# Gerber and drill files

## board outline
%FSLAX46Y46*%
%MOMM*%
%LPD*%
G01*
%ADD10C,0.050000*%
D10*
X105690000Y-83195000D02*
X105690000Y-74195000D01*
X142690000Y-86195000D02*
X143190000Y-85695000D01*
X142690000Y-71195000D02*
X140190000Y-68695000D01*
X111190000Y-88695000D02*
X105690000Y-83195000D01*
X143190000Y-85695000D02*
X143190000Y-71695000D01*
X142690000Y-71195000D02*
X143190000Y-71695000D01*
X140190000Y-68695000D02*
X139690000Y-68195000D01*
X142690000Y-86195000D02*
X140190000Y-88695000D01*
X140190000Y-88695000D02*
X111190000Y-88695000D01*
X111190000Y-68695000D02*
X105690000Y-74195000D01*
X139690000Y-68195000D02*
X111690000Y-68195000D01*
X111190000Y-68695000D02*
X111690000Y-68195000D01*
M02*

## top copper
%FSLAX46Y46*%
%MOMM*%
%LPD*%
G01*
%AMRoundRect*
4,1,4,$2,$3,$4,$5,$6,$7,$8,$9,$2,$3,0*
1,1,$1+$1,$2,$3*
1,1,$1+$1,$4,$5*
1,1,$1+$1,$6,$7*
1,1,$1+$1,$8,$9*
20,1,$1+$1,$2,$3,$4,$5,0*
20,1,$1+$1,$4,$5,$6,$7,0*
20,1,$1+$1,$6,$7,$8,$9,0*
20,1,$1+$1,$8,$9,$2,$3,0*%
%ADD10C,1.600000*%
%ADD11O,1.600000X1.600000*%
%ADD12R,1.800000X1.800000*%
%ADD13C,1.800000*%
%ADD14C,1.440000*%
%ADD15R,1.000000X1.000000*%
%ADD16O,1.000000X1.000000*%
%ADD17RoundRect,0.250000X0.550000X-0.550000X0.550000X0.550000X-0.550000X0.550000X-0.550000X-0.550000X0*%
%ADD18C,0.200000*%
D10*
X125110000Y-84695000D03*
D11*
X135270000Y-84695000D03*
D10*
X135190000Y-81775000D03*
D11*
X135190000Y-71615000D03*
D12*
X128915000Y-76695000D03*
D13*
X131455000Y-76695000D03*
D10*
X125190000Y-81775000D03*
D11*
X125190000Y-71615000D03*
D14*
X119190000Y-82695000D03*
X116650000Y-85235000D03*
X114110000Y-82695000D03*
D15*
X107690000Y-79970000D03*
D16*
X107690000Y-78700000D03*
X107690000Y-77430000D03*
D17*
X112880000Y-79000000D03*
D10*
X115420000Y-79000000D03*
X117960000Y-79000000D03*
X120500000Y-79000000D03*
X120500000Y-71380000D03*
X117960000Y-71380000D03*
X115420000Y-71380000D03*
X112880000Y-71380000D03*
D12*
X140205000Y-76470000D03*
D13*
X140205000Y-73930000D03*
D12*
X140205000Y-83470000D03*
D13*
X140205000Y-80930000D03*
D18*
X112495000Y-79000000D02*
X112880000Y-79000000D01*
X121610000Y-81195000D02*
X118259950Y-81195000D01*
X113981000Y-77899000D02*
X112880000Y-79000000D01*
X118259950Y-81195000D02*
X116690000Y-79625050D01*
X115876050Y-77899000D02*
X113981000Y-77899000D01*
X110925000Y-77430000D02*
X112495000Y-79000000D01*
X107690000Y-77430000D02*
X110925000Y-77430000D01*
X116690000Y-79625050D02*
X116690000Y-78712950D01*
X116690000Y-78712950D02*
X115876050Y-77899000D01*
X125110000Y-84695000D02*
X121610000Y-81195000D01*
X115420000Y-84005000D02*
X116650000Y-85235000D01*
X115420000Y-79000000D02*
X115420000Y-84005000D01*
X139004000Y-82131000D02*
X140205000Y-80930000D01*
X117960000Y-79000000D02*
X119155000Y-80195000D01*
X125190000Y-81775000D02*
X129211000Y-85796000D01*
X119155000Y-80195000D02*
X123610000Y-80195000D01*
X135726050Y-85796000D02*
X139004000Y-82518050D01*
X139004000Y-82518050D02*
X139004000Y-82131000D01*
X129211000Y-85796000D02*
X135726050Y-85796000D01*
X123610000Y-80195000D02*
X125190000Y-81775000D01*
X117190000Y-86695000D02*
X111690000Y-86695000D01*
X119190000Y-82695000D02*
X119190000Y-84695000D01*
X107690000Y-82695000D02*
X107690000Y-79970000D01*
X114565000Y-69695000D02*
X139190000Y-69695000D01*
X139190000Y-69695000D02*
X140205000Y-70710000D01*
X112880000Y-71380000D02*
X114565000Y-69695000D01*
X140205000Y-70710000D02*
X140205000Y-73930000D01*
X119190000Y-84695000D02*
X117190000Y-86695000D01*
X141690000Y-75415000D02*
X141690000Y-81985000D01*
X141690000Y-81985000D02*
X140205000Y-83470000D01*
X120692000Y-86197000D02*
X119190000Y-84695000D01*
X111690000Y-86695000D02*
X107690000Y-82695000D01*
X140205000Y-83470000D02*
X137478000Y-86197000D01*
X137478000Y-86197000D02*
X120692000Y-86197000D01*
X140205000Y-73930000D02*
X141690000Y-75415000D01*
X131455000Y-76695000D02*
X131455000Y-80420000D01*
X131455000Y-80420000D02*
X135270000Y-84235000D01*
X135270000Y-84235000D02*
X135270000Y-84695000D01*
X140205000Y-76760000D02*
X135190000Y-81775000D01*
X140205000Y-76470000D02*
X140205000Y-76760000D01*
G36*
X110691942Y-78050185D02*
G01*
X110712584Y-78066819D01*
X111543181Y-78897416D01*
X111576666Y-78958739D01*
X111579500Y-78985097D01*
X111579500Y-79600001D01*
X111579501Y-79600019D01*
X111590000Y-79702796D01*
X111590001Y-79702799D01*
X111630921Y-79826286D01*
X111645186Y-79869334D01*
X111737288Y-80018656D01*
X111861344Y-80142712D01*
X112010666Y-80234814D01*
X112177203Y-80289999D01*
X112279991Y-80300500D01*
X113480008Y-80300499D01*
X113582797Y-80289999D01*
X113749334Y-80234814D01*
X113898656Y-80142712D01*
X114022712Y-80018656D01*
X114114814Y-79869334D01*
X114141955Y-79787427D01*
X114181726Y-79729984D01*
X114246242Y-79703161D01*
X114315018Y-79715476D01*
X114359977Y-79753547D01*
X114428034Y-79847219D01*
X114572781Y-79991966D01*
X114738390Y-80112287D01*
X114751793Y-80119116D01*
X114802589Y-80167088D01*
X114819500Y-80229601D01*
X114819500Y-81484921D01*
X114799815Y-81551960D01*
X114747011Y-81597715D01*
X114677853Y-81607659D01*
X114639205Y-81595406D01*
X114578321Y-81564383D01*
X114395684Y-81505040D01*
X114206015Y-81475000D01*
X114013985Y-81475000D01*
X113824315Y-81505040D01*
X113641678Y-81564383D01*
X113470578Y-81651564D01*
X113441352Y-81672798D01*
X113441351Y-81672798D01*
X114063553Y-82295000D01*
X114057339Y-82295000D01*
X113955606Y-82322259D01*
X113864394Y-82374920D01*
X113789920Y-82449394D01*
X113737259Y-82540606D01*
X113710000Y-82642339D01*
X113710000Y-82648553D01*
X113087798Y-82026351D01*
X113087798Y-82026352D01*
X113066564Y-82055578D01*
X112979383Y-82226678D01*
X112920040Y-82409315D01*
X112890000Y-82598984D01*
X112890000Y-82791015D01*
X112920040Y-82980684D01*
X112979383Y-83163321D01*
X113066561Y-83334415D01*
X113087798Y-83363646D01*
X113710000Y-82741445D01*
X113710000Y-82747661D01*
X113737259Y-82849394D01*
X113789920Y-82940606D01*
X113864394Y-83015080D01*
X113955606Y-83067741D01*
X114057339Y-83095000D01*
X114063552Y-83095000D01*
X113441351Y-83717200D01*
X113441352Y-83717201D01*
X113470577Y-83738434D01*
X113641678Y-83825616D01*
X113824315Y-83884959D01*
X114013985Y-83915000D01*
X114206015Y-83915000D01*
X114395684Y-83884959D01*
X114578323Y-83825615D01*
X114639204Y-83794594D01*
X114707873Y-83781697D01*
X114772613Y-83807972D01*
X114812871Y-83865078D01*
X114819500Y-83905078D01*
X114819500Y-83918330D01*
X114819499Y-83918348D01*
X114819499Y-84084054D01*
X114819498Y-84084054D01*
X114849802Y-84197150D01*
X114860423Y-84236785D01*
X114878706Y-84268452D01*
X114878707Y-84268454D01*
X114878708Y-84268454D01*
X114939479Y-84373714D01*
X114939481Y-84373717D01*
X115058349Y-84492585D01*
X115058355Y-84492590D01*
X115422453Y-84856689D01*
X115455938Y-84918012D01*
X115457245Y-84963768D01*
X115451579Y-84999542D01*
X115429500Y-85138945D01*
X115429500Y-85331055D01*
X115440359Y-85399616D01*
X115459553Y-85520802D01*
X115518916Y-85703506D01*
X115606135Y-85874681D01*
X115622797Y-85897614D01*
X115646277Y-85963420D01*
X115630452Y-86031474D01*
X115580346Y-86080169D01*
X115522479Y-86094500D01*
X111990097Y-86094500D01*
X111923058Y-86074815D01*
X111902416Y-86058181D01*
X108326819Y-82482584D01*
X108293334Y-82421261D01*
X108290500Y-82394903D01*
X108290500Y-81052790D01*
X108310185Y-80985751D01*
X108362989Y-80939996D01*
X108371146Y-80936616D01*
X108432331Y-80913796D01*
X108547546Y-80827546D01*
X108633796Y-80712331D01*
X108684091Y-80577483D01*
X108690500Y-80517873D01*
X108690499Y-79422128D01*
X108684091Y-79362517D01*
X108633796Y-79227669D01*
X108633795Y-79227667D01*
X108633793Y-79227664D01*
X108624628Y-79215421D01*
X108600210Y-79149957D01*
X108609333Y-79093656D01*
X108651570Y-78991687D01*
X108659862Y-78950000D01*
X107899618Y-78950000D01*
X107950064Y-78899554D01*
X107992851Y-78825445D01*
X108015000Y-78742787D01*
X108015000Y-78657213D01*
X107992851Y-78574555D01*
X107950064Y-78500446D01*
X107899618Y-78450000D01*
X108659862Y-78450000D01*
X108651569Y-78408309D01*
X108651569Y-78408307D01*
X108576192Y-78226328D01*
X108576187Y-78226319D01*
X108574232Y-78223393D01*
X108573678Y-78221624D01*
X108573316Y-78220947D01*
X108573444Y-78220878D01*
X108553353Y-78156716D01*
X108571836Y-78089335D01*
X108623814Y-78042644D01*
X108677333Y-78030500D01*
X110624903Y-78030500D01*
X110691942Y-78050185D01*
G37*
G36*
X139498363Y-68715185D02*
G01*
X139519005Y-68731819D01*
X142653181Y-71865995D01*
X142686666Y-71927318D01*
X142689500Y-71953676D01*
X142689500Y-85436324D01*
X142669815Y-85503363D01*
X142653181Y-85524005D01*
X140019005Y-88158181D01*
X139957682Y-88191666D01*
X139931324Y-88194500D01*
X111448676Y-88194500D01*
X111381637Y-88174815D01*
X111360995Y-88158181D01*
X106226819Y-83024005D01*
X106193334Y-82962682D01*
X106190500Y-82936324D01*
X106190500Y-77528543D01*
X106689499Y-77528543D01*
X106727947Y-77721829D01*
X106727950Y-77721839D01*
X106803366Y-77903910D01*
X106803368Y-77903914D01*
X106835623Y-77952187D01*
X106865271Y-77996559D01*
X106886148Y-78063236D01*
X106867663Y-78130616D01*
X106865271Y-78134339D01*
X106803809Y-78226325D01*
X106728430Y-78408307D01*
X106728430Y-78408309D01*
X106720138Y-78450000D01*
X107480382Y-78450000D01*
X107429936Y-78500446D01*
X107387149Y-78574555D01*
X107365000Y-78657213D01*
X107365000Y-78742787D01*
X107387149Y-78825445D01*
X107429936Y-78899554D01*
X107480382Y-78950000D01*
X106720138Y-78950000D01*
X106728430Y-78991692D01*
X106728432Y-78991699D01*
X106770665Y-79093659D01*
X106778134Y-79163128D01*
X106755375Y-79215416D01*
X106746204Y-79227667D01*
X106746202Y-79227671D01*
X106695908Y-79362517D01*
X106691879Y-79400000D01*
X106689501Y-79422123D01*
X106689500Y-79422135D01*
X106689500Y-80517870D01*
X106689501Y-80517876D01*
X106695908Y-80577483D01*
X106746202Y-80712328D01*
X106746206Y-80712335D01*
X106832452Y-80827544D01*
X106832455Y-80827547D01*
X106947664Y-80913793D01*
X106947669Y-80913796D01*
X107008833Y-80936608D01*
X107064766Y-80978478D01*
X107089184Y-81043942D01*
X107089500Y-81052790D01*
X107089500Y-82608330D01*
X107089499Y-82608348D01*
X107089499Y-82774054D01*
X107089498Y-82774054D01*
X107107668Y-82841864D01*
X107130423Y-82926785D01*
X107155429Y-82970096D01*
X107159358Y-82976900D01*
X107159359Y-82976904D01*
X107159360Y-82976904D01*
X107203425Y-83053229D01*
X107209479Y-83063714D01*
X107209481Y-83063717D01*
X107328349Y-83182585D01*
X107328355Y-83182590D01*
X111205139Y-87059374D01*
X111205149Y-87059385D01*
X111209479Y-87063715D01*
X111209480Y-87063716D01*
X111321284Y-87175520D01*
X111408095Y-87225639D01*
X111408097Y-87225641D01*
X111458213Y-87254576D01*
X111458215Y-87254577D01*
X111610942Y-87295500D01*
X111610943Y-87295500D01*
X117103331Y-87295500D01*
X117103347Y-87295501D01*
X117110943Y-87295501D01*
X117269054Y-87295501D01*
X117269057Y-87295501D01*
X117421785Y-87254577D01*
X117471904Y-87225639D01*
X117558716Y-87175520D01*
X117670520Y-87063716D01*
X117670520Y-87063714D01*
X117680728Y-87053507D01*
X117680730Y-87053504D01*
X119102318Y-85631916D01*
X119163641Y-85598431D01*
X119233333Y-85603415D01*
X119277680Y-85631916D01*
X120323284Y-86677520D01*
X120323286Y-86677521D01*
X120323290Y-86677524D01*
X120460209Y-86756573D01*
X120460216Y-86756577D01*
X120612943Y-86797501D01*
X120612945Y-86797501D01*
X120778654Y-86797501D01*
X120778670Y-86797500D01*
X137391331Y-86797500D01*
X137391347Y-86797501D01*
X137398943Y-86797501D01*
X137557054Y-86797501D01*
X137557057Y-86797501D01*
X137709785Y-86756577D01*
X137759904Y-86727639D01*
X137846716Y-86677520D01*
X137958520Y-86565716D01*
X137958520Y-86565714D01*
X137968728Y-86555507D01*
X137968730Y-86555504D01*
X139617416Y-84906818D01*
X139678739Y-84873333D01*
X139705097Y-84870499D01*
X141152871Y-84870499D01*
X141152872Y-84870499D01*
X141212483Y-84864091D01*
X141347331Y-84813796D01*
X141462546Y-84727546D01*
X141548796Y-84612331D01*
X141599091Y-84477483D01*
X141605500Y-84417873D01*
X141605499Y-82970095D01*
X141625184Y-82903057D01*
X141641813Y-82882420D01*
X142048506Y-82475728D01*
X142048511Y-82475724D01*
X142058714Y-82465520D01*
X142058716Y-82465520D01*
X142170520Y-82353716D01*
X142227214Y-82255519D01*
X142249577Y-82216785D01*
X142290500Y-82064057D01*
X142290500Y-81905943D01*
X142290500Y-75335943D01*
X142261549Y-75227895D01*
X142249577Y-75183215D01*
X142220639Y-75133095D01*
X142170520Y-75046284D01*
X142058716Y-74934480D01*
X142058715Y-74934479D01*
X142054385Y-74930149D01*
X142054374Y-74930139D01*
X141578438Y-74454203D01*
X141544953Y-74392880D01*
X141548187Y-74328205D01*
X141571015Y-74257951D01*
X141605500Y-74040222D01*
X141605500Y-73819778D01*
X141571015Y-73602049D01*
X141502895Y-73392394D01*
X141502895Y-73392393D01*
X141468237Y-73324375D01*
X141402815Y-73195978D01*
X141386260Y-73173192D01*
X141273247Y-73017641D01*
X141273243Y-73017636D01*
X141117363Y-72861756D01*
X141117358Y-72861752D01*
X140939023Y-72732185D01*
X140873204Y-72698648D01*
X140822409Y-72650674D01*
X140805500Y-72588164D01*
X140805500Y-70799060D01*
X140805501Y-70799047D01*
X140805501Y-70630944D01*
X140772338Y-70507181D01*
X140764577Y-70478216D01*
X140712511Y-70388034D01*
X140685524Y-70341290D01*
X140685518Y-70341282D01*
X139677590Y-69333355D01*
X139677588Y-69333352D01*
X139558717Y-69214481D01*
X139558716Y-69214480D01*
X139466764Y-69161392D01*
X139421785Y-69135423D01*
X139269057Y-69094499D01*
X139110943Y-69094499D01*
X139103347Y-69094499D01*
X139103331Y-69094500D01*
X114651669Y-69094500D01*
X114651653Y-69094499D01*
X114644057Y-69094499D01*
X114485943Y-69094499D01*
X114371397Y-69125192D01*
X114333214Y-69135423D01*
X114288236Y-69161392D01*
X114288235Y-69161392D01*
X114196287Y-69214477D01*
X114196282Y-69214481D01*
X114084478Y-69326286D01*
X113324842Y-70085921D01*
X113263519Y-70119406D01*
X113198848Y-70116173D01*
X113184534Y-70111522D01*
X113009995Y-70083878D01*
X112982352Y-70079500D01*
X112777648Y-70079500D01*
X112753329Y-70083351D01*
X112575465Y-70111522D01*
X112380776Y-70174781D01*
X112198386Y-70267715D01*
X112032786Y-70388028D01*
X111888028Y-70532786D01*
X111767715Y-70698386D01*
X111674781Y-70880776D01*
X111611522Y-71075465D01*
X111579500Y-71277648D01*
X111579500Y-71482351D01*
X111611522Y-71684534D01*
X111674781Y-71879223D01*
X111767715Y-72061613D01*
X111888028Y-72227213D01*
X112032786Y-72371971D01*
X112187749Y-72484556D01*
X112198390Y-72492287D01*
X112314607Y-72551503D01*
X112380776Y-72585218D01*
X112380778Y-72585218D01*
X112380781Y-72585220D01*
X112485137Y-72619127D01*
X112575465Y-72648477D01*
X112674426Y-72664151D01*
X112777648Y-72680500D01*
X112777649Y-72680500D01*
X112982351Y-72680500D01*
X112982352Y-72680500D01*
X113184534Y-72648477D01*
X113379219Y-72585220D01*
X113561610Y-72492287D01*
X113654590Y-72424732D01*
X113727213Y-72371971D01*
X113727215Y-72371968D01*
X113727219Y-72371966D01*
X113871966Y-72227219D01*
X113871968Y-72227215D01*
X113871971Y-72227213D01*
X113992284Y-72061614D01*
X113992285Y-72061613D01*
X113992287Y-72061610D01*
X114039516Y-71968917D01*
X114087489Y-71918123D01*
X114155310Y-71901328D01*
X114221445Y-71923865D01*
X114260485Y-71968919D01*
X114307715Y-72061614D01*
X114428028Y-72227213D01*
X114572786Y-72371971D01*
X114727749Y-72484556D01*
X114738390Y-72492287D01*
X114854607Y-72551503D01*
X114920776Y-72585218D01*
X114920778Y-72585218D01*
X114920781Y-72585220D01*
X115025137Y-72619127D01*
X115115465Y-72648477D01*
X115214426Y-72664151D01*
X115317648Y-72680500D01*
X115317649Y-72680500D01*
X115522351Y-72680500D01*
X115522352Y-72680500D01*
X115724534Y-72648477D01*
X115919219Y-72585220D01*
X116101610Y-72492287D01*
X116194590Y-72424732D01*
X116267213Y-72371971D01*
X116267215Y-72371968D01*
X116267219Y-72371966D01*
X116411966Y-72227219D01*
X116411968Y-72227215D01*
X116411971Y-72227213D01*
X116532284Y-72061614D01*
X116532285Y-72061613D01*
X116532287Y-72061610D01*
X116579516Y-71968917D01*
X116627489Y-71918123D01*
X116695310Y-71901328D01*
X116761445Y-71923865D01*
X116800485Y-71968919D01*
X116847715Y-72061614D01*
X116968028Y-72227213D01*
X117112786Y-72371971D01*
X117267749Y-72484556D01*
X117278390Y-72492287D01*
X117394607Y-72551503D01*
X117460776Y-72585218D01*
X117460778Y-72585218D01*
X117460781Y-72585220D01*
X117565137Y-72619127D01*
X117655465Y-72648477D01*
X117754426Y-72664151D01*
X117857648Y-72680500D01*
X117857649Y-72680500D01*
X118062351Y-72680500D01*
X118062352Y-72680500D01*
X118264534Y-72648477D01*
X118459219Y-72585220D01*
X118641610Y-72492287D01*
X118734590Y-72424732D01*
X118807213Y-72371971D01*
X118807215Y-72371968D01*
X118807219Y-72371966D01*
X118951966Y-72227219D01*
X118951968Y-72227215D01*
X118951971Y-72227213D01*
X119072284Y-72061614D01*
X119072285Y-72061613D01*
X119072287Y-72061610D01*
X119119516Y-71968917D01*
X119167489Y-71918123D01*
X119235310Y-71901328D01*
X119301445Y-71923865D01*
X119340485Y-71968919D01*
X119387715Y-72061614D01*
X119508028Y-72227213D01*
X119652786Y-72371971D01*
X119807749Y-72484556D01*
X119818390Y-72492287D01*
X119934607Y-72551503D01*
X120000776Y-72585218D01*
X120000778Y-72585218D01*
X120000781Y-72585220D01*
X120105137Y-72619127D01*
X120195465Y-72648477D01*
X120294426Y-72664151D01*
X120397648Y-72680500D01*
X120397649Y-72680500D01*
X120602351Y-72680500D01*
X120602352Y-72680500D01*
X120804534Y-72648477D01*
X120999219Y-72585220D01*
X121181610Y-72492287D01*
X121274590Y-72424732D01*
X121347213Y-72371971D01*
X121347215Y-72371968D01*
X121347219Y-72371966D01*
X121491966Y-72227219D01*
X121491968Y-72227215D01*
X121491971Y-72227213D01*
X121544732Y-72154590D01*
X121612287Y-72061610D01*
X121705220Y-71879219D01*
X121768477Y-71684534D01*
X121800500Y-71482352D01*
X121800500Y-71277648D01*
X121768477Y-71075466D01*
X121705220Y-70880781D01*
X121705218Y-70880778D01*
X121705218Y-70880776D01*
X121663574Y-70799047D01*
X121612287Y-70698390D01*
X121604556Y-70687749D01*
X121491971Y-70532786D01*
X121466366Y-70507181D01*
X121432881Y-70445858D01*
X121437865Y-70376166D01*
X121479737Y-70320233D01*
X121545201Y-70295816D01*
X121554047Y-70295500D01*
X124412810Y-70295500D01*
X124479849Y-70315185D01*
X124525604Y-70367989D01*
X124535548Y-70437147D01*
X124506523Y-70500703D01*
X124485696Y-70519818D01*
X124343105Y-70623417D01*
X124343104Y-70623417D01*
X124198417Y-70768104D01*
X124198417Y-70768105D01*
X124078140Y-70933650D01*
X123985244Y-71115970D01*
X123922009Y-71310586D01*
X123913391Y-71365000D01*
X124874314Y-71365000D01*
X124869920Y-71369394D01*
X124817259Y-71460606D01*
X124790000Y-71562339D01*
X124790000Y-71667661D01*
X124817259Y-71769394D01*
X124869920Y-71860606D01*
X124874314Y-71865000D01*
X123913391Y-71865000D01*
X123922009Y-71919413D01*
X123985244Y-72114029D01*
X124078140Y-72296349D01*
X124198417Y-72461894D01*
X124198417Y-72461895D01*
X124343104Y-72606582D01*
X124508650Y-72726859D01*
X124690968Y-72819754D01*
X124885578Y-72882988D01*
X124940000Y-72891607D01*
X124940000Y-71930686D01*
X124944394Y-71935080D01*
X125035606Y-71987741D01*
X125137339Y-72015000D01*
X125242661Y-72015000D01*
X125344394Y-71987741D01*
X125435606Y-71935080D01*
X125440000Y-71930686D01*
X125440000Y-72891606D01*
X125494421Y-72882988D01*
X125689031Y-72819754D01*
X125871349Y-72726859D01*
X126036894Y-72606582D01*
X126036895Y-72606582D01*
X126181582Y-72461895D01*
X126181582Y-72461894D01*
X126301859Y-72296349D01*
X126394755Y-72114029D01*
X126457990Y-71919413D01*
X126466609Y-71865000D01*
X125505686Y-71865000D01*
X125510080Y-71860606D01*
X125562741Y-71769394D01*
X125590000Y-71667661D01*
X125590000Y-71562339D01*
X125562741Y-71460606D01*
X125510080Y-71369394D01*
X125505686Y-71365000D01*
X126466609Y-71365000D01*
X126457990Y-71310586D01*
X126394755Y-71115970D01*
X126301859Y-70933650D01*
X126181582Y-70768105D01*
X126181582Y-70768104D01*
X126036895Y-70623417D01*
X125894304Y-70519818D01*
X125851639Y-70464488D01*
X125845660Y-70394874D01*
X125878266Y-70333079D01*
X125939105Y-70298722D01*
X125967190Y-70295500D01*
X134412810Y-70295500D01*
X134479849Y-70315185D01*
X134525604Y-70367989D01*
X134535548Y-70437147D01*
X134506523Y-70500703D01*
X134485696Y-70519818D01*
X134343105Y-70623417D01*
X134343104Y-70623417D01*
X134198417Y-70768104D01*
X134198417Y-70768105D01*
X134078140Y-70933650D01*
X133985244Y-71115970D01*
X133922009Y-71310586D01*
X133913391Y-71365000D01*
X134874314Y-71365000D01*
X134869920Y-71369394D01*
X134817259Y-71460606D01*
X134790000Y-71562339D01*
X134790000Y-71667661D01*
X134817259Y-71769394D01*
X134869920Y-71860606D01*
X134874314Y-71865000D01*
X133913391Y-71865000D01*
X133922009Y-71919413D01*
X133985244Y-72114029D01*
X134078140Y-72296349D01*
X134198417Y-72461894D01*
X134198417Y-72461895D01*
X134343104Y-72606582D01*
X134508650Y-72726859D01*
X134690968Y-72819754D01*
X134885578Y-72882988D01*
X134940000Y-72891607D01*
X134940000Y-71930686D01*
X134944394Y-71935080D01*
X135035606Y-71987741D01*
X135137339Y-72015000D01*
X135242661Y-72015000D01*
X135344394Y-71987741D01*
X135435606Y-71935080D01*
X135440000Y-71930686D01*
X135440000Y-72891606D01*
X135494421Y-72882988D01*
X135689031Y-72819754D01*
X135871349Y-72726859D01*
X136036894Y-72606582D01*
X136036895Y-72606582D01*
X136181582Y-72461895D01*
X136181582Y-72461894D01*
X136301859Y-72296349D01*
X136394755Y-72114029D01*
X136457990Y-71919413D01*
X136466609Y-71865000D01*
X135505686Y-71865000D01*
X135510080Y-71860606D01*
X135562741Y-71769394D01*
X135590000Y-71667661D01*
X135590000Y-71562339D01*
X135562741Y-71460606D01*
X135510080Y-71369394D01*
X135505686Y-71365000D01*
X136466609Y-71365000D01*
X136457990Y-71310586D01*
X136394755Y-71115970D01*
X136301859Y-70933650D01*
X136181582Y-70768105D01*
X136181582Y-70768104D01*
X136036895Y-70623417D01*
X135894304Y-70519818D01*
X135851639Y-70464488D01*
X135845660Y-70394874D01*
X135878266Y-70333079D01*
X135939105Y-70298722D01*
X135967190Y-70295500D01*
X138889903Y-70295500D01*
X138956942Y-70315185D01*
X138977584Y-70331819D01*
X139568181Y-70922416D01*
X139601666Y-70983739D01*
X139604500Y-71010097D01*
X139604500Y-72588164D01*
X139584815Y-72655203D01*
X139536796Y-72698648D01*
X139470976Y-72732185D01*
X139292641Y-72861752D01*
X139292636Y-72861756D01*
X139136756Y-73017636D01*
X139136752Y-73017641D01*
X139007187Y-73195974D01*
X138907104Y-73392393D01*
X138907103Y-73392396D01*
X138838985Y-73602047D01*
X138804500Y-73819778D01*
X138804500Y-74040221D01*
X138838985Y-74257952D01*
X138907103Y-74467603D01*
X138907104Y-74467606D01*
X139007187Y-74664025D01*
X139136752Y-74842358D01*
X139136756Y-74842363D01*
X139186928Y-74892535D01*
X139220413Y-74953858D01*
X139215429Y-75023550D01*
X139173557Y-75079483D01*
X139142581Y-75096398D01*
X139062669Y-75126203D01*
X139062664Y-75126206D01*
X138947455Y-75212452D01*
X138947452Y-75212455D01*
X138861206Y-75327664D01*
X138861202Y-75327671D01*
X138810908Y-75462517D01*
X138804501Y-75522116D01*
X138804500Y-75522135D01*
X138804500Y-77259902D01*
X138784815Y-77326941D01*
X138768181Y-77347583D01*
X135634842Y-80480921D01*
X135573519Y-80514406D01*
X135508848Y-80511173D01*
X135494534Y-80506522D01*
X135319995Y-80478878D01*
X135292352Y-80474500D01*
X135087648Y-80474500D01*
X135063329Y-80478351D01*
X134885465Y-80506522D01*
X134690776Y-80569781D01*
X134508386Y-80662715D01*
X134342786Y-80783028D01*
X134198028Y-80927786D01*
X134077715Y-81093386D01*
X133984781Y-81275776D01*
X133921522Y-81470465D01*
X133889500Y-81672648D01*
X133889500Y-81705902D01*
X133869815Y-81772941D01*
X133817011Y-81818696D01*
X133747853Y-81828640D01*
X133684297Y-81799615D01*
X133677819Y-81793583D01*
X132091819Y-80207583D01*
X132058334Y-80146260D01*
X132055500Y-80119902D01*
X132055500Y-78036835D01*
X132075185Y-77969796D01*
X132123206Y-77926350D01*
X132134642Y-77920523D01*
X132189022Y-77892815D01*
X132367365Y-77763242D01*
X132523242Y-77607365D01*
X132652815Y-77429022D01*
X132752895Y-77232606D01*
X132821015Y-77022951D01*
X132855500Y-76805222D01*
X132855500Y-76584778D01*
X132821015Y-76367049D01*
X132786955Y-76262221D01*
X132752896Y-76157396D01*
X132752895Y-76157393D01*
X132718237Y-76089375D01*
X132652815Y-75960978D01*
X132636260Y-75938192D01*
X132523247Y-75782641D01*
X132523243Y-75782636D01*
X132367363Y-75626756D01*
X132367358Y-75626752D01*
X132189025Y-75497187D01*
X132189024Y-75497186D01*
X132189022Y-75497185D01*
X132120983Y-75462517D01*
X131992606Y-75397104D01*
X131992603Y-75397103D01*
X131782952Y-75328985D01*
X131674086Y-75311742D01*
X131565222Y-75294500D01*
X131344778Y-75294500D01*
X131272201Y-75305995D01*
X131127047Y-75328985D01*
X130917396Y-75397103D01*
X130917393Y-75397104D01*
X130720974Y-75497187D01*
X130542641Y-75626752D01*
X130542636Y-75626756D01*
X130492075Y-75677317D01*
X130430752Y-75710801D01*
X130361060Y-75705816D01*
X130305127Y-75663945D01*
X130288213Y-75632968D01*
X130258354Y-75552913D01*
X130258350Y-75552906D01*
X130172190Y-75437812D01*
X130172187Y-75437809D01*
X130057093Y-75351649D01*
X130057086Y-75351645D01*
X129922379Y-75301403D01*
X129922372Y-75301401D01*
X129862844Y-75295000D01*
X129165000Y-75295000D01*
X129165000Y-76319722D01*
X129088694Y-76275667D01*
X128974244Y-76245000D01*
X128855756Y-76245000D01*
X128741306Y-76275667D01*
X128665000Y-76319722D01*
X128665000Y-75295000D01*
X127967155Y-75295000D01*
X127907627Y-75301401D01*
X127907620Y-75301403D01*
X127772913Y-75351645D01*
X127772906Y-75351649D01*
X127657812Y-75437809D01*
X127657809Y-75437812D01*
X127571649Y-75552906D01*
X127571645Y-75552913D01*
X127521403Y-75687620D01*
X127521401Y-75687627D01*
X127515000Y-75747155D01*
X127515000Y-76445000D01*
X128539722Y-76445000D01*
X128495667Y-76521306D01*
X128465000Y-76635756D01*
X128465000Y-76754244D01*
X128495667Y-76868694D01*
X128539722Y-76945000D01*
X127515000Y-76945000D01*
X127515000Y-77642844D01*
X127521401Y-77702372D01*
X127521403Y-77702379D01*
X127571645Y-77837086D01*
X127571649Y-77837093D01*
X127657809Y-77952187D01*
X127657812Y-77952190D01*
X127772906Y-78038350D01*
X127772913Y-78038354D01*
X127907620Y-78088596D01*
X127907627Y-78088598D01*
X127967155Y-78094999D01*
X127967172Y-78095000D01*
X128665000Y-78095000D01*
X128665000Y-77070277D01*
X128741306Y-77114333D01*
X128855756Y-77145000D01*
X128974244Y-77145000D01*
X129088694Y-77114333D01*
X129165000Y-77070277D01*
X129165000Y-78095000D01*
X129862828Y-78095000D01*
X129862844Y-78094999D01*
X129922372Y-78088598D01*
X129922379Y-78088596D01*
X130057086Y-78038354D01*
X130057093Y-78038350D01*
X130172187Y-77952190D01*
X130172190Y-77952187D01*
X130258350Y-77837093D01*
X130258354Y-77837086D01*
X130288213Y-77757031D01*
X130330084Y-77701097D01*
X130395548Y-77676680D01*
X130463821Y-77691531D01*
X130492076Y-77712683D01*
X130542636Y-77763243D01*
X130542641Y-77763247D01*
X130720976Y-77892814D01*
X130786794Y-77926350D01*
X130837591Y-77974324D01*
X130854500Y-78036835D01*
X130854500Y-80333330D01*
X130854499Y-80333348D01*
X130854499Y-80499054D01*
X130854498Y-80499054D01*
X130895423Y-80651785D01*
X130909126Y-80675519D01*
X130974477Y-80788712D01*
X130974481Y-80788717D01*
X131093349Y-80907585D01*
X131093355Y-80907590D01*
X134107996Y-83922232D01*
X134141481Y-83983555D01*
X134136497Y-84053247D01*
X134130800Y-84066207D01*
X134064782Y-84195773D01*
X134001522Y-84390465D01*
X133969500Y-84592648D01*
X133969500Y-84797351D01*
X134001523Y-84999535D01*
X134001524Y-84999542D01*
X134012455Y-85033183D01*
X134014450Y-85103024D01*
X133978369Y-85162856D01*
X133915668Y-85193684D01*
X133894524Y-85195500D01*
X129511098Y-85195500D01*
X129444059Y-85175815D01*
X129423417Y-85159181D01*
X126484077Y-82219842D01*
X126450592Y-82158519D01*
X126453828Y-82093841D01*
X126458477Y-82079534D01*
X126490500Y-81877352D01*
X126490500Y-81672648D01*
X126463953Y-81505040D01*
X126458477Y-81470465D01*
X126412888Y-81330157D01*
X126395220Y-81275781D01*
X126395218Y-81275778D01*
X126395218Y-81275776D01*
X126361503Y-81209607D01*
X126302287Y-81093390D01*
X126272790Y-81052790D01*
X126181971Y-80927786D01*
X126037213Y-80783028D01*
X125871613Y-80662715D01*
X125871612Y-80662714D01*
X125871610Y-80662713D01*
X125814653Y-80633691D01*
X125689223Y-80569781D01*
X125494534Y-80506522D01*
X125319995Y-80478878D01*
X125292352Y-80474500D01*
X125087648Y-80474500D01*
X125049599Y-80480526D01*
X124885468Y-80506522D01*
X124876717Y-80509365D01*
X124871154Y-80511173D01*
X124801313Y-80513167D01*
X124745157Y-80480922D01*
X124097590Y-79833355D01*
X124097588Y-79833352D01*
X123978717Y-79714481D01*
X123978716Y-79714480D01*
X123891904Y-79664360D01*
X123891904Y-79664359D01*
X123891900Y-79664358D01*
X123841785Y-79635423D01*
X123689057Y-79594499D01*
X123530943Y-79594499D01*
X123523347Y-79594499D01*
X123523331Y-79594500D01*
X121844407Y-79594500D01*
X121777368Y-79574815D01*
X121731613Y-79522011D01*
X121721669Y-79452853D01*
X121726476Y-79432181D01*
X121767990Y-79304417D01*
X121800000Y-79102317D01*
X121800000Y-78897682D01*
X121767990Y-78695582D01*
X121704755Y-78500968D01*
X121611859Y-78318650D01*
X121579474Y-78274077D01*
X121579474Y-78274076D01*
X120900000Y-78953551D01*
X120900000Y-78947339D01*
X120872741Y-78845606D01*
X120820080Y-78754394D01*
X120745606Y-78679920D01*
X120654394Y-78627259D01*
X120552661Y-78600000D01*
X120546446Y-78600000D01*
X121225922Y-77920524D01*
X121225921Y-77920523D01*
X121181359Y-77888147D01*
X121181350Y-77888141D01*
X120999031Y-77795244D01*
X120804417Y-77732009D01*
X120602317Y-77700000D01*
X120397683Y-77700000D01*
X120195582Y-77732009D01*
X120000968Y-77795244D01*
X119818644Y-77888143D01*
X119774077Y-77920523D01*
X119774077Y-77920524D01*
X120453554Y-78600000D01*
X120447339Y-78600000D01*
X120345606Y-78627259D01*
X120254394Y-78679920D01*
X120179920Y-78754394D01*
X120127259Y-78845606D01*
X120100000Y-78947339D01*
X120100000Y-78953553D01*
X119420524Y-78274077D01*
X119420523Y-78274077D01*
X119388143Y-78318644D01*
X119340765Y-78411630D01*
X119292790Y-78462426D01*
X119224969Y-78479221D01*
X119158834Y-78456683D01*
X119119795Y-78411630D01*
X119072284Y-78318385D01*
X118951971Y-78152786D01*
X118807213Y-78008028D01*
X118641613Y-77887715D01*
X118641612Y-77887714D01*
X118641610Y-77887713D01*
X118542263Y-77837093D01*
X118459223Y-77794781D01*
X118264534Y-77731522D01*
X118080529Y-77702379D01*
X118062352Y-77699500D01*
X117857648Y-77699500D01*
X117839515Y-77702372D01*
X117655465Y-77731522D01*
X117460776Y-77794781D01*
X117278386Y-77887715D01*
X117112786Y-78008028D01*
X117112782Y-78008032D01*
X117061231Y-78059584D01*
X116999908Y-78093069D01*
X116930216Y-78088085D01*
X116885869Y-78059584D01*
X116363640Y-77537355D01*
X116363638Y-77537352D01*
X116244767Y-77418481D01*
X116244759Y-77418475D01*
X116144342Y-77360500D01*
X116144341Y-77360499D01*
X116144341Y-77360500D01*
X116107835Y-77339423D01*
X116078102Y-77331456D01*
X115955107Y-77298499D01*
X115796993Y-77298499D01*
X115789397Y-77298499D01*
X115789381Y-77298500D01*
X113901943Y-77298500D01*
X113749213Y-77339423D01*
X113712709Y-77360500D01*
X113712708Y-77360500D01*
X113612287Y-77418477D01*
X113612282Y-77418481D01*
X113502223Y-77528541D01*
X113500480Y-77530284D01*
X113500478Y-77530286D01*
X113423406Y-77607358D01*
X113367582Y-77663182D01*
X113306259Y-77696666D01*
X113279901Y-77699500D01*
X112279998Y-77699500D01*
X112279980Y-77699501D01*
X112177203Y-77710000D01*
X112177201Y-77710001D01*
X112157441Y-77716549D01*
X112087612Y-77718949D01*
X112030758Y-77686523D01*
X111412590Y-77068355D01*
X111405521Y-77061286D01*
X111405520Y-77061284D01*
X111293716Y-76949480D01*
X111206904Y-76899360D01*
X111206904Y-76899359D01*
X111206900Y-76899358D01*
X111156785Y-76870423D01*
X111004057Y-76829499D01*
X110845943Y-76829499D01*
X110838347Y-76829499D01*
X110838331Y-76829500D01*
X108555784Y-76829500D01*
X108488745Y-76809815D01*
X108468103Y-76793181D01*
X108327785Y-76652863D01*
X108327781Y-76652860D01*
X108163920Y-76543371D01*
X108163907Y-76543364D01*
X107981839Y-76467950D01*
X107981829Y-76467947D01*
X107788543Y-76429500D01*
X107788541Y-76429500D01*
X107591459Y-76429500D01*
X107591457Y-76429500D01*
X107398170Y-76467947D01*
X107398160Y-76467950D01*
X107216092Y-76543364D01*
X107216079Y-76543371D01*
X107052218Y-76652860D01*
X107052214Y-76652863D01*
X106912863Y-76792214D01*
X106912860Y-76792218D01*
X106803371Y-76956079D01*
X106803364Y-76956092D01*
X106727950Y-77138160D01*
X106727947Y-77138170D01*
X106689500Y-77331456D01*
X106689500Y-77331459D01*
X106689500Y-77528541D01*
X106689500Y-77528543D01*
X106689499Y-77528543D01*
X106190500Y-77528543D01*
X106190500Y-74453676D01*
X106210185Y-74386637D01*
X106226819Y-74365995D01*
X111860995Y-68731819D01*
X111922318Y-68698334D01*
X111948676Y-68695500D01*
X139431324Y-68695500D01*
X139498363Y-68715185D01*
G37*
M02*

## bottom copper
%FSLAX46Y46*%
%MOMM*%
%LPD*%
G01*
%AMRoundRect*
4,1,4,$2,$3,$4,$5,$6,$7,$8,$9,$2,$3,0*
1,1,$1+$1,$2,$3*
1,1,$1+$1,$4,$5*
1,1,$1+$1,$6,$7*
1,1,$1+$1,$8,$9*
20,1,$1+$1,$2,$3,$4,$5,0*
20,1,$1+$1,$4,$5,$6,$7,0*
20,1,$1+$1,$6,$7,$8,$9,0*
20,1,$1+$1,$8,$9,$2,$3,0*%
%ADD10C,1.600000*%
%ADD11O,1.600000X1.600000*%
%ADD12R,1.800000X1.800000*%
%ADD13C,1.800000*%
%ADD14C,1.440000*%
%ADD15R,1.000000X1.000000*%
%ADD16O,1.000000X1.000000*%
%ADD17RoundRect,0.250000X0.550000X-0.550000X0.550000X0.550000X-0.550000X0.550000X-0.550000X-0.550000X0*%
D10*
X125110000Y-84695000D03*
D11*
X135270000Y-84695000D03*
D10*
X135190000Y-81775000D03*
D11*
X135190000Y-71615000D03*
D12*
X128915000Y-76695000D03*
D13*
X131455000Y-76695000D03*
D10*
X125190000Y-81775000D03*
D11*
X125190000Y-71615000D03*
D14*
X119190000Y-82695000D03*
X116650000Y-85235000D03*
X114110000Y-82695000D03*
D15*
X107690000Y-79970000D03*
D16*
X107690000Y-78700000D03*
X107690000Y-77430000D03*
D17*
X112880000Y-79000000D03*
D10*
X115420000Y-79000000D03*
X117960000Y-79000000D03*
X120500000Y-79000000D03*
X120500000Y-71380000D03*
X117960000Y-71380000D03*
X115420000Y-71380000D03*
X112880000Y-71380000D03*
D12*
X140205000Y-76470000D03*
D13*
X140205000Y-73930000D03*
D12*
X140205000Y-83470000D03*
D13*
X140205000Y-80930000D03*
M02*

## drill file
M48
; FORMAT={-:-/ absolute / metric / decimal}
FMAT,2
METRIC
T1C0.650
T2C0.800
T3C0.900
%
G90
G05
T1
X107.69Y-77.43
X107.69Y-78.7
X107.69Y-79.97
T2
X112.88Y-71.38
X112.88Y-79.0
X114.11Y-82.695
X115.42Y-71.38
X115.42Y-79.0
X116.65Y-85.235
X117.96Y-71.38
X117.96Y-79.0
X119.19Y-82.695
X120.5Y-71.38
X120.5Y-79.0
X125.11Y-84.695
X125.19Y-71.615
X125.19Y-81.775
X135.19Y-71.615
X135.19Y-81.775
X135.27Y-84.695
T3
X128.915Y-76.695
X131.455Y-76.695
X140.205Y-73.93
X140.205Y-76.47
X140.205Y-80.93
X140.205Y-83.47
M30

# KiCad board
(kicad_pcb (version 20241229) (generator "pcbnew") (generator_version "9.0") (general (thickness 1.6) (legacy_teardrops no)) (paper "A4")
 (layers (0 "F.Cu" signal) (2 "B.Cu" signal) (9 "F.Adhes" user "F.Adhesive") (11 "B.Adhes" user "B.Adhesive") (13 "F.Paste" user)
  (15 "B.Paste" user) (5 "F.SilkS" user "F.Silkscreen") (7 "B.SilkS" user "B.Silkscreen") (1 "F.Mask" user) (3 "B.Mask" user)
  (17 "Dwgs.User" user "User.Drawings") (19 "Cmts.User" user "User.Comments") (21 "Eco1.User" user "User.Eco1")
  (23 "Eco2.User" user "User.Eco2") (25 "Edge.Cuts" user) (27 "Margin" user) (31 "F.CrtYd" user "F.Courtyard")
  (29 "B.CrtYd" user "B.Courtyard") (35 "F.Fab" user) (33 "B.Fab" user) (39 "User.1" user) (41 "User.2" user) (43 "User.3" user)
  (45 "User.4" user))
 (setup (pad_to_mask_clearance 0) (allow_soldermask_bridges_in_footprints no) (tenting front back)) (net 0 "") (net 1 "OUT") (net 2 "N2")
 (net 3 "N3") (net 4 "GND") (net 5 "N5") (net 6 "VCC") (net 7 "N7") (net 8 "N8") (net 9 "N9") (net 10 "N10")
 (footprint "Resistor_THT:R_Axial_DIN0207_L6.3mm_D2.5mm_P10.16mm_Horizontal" (layer "F.Cu") (at 125.11 84.695)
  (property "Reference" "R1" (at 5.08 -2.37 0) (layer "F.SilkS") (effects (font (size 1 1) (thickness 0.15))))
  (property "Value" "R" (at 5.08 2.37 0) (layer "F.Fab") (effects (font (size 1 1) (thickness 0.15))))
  (pad "1" thru_hole circle (at 0 0) (size 1.6 1.6) (drill 0.8) (layers "*.Cu" "*.Mask") (remove_unused_layers no) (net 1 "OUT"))
  (pad "2" thru_hole oval (at 10.16 0) (size 1.6 1.6) (drill 0.8) (layers "*.Cu" "*.Mask") (remove_unused_layers no) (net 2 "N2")))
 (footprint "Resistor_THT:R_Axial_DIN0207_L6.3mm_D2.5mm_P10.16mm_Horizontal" (layer "F.Cu") (at 135.19 81.775 90)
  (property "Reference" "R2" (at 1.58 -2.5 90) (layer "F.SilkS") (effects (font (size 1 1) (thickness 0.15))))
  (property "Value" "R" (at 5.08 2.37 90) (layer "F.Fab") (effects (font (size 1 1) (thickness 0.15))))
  (pad "1" thru_hole circle (at 0 0 90) (size 1.6 1.6) (drill 0.8) (layers "*.Cu" "*.Mask") (remove_unused_layers no) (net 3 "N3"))
  (pad "2" thru_hole oval (at 10.16 0 90) (size 1.6 1.6) (drill 0.8) (layers "*.Cu" "*.Mask") (remove_unused_layers no) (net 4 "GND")))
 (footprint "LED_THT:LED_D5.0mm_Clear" (layer "F.Cu") (at 128.915 76.695)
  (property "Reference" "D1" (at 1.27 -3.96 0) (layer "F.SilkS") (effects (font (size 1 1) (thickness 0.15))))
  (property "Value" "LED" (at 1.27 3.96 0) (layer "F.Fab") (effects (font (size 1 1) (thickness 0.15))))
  (pad "1" thru_hole rect (at 0 0) (size 1.8 1.8) (drill 0.9) (layers "*.Cu" "*.Mask") (remove_unused_layers no) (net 4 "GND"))
  (pad "2" thru_hole circle (at 2.54 0) (size 1.8 1.8) (drill 0.9) (layers "*.Cu" "*.Mask") (remove_unused_layers no) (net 2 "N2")))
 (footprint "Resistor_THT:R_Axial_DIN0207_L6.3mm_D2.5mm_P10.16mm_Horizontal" (layer "F.Cu") (at 125.19 81.775 90)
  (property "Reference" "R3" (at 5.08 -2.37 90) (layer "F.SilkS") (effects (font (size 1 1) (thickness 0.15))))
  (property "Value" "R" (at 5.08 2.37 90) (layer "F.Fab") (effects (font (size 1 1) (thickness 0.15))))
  (pad "1" thru_hole circle (at 0 0 90) (size 1.6 1.6) (drill 0.8) (layers "*.Cu" "*.Mask") (remove_unused_layers no) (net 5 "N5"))
  (pad "2" thru_hole oval (at 10.16 0 90) (size 1.6 1.6) (drill 0.8) (layers "*.Cu" "*.Mask") (remove_unused_layers no) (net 4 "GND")))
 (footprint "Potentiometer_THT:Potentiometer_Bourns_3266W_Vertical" (layer "F.Cu") (at 119.19 82.695)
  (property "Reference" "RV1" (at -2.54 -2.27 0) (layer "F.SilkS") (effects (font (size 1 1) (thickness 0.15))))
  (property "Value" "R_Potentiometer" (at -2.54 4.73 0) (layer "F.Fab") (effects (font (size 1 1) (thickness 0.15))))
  (pad "1" thru_hole circle (at 0 0) (size 1.44 1.44) (drill 0.8) (layers "*.Cu" "*.Mask") (remove_unused_layers no) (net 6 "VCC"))
  (pad "2" thru_hole circle (at -2.54 2.54) (size 1.44 1.44) (drill 0.8) (layers "*.Cu" "*.Mask") (remove_unused_layers no) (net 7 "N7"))
  (pad "3" thru_hole circle (at -5.08 0) (size 1.44 1.44) (drill 0.8) (layers "*.Cu" "*.Mask") (remove_unused_layers no) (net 4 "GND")))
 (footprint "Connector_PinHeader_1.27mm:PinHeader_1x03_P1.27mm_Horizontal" (layer "F.Cu") (at 107.69 79.97 180)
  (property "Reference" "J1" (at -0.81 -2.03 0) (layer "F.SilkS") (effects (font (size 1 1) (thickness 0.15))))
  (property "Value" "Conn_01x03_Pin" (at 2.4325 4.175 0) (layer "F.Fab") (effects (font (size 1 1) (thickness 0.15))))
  (pad "1" thru_hole rect (at 0 0 180) (size 1 1) (drill 0.65) (layers "*.Cu" "*.Mask") (remove_unused_layers no) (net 6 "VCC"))
  (pad "2" thru_hole oval (at 0 1.27 180) (size 1 1) (drill 0.65) (layers "*.Cu" "*.Mask") (remove_unused_layers no) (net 4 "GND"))
  (pad "3" thru_hole oval (at 0 2.54 180) (size 1 1) (drill 0.65) (layers "*.Cu" "*.Mask") (remove_unused_layers no) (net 1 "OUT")))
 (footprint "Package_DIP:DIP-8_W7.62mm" (layer "F.Cu") (at 112.88 79 90)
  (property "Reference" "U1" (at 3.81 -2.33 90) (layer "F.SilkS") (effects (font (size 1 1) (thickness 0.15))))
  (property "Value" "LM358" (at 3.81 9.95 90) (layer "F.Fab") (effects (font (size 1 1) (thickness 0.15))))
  (pad "1" thru_hole roundrect (at 0 0 90) (size 1.6 1.6) (drill 0.8) (layers "*.Cu" "*.Mask") (remove_unused_layers no)
   (roundrect_rratio 0.15625) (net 1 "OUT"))
  (pad "2" thru_hole circle (at 0 2.54 90) (size 1.6 1.6) (drill 0.8) (layers "*.Cu" "*.Mask") (remove_unused_layers no) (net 7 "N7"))
  (pad "3" thru_hole circle (at 0 5.08 90) (size 1.6 1.6) (drill 0.8) (layers "*.Cu" "*.Mask") (remove_unused_layers no) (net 5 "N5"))
  (pad "4" thru_hole circle (at 0 7.62 90) (size 1.6 1.6) (drill 0.8) (layers "*.Cu" "*.Mask") (remove_unused_layers no) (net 4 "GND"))
  (pad "5" thru_hole circle (at 7.62 7.62 90) (size 1.6 1.6) (drill 0.8) (layers "*.Cu" "*.Mask") (remove_unused_layers no) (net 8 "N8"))
  (pad "6" thru_hole circle (at 7.62 5.08 90) (size 1.6 1.6) (drill 0.8) (layers "*.Cu" "*.Mask") (remove_unused_layers no) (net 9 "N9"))
  (pad "7" thru_hole circle (at 7.62 2.54 90) (size 1.6 1.6) (drill 0.8) (layers "*.Cu" "*.Mask") (remove_unused_layers no) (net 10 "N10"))
  (pad "8" thru_hole circle (at 7.62 0 90) (size 1.6 1.6) (drill 0.8) (layers "*.Cu" "*.Mask") (remove_unused_layers no) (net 6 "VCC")))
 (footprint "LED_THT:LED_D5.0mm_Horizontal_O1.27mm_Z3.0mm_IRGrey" (layer "F.Cu") (at 140.205 76.47 90)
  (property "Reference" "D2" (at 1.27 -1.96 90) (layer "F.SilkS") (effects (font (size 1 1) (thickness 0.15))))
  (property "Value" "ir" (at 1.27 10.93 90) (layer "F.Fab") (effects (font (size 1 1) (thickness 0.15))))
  (pad "1" thru_hole rect (at 0 0 90) (size 1.8 1.8) (drill 0.9) (layers "*.Cu" "*.Mask") (remove_unused_layers no) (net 3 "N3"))
  (pad "2" thru_hole circle (at 2.54 0 90) (size 1.8 1.8) (drill 0.9) (layers "*.Cu" "*.Mask") (remove_unused_layers no) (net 6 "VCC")))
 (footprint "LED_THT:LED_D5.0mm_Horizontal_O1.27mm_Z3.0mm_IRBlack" (layer "F.Cu") (at 140.205 83.47 90)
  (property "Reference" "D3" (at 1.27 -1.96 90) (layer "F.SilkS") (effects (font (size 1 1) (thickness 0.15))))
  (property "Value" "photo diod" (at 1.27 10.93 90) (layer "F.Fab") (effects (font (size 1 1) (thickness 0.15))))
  (pad "1" thru_hole rect (at 0 0 90) (size 1.8 1.8) (drill 0.9) (layers "*.Cu" "*.Mask") (remove_unused_layers no) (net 6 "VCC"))
  (pad "2" thru_hole circle (at 2.54 0 90) (size 1.8 1.8) (drill 0.9) (layers "*.Cu" "*.Mask") (remove_unused_layers no) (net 5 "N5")))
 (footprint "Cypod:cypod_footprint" (layer "B.Cu") (at 117 82.5 180)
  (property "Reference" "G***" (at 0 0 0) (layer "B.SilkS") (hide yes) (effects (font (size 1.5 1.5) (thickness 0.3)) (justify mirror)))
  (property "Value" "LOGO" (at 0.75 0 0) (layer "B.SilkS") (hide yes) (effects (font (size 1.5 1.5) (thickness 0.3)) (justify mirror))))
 (gr_line (start 105.69 83.195) (end 105.69 74.195) (stroke (width 0.05) (type default)) (layer "Edge.Cuts"))
 (gr_line (start 142.69 86.195) (end 143.19 85.695) (stroke (width 0.05) (type default)) (layer "Edge.Cuts"))
 (gr_line (start 142.69 71.195) (end 140.19 68.695) (stroke (width 0.05) (type default)) (layer "Edge.Cuts"))
 (gr_line (start 111.19 88.695) (end 105.69 83.195) (stroke (width 0.05) (type default)) (layer "Edge.Cuts"))
 (gr_line (start 143.19 85.695) (end 143.19 71.695) (stroke (width 0.05) (type default)) (layer "Edge.Cuts"))
 (gr_line (start 142.69 71.195) (end 143.19 71.695) (stroke (width 0.05) (type default)) (layer "Edge.Cuts"))
 (gr_line (start 140.19 68.695) (end 139.69 68.195) (stroke (width 0.05) (type default)) (layer "Edge.Cuts"))
 (gr_line (start 142.69 86.195) (end 140.19 88.695) (stroke (width 0.05) (type default)) (layer "Edge.Cuts"))
 (gr_line (start 140.19 88.695) (end 111.19 88.695) (stroke (width 0.05) (type default)) (layer "Edge.Cuts"))
 (gr_line (start 111.19 68.695) (end 105.69 74.195) (stroke (width 0.05) (type default)) (layer "Edge.Cuts"))
 (gr_line (start 139.69 68.195) (end 111.69 68.195) (stroke (width 0.05) (type default)) (layer "Edge.Cuts"))
 (gr_line (start 111.19 68.695) (end 111.69 68.195) (stroke (width 0.05) (type default)) (layer "Edge.Cuts"))
 (segment (start 112.495 79) (end 112.88 79) (width 0.2) (layer "F.Cu") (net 1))
 (segment (start 121.61 81.195) (end 118.25995 81.195) (width 0.2) (layer "F.Cu") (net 1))
 (segment (start 113.981 77.899) (end 112.88 79) (width 0.2) (layer "F.Cu") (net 1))
 (segment (start 118.25995 81.195) (end 116.69 79.62505) (width 0.2) (layer "F.Cu") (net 1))
 (segment (start 115.87605 77.899) (end 113.981 77.899) (width 0.2) (layer "F.Cu") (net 1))
 (segment (start 110.925 77.43) (end 112.495 79) (width 0.2) (layer "F.Cu") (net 1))
 (segment (start 107.69 77.43) (end 110.925 77.43) (width 0.2) (layer "F.Cu") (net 1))
 (segment (start 116.69 79.62505) (end 116.69 78.71295) (width 0.2) (layer "F.Cu") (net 1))
 (segment (start 116.69 78.71295) (end 115.87605 77.899) (width 0.2) (layer "F.Cu") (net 1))
 (segment (start 125.11 84.695) (end 121.61 81.195) (width 0.2) (layer "F.Cu") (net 1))
 (segment (start 115.42 84.005) (end 116.65 85.235) (width 0.2) (layer "F.Cu") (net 7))
 (segment (start 115.42 79) (end 115.42 84.005) (width 0.2) (layer "F.Cu") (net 7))
 (segment (start 139.004 82.131) (end 140.205 80.93) (width 0.2) (layer "F.Cu") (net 5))
 (segment (start 117.96 79) (end 119.155 80.195) (width 0.2) (layer "F.Cu") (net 5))
 (segment (start 125.19 81.775) (end 129.211 85.796) (width 0.2) (layer "F.Cu") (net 5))
 (segment (start 119.155 80.195) (end 123.61 80.195) (width 0.2) (layer "F.Cu") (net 5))
 (segment (start 135.72605 85.796) (end 139.004 82.51805) (width 0.2) (layer "F.Cu") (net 5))
 (segment (start 139.004 82.51805) (end 139.004 82.131) (width 0.2) (layer "F.Cu") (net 5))
 (segment (start 129.211 85.796) (end 135.72605 85.796) (width 0.2) (layer "F.Cu") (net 5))
 (segment (start 123.61 80.195) (end 125.19 81.775) (width 0.2) (layer "F.Cu") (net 5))
 (segment (start 117.19 86.695) (end 111.69 86.695) (width 0.2) (layer "F.Cu") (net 6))
 (segment (start 119.19 82.695) (end 119.19 84.695) (width 0.2) (layer "F.Cu") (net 6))
 (segment (start 107.69 82.695) (end 107.69 79.97) (width 0.2) (layer "F.Cu") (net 6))
 (segment (start 114.565 69.695) (end 139.19 69.695) (width 0.2) (layer "F.Cu") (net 6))
 (segment (start 139.19 69.695) (end 140.205 70.71) (width 0.2) (layer "F.Cu") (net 6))
 (segment (start 112.88 71.38) (end 114.565 69.695) (width 0.2) (layer "F.Cu") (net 6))
 (segment (start 140.205 70.71) (end 140.205 73.93) (width 0.2) (layer "F.Cu") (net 6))
 (segment (start 119.19 84.695) (end 117.19 86.695) (width 0.2) (layer "F.Cu") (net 6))
 (segment (start 141.69 75.415) (end 141.69 81.985) (width 0.2) (layer "F.Cu") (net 6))
 (segment (start 141.69 81.985) (end 140.205 83.47) (width 0.2) (layer "F.Cu") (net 6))
 (segment (start 120.692 86.197) (end 119.19 84.695) (width 0.2) (layer "F.Cu") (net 6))
 (segment (start 111.69 86.695) (end 107.69 82.695) (width 0.2) (layer "F.Cu") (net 6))
 (segment (start 140.205 83.47) (end 137.478 86.197) (width 0.2) (layer "F.Cu") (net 6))
 (segment (start 137.478 86.197) (end 120.692 86.197) (width 0.2) (layer "F.Cu") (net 6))
 (segment (start 140.205 73.93) (end 141.69 75.415) (width 0.2) (layer "F.Cu") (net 6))
 (segment (start 131.455 76.695) (end 131.455 80.42) (width 0.2) (layer "F.Cu") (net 2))
 (segment (start 131.455 80.42) (end 135.27 84.235) (width 0.2) (layer "F.Cu") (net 2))
 (segment (start 135.27 84.235) (end 135.27 84.695) (width 0.2) (layer "F.Cu") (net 2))
 (segment (start 140.205 76.76) (end 135.19 81.775) (width 0.2) (layer "F.Cu") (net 3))
 (segment (start 140.205 76.47) (end 140.205 76.76) (width 0.2) (layer "F.Cu") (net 3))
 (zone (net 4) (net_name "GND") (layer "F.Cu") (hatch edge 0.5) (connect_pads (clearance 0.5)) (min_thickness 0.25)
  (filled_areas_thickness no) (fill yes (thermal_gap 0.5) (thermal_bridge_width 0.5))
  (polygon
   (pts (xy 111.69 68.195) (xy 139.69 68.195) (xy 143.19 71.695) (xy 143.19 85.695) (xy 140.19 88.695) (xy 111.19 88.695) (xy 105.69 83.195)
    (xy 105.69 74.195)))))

